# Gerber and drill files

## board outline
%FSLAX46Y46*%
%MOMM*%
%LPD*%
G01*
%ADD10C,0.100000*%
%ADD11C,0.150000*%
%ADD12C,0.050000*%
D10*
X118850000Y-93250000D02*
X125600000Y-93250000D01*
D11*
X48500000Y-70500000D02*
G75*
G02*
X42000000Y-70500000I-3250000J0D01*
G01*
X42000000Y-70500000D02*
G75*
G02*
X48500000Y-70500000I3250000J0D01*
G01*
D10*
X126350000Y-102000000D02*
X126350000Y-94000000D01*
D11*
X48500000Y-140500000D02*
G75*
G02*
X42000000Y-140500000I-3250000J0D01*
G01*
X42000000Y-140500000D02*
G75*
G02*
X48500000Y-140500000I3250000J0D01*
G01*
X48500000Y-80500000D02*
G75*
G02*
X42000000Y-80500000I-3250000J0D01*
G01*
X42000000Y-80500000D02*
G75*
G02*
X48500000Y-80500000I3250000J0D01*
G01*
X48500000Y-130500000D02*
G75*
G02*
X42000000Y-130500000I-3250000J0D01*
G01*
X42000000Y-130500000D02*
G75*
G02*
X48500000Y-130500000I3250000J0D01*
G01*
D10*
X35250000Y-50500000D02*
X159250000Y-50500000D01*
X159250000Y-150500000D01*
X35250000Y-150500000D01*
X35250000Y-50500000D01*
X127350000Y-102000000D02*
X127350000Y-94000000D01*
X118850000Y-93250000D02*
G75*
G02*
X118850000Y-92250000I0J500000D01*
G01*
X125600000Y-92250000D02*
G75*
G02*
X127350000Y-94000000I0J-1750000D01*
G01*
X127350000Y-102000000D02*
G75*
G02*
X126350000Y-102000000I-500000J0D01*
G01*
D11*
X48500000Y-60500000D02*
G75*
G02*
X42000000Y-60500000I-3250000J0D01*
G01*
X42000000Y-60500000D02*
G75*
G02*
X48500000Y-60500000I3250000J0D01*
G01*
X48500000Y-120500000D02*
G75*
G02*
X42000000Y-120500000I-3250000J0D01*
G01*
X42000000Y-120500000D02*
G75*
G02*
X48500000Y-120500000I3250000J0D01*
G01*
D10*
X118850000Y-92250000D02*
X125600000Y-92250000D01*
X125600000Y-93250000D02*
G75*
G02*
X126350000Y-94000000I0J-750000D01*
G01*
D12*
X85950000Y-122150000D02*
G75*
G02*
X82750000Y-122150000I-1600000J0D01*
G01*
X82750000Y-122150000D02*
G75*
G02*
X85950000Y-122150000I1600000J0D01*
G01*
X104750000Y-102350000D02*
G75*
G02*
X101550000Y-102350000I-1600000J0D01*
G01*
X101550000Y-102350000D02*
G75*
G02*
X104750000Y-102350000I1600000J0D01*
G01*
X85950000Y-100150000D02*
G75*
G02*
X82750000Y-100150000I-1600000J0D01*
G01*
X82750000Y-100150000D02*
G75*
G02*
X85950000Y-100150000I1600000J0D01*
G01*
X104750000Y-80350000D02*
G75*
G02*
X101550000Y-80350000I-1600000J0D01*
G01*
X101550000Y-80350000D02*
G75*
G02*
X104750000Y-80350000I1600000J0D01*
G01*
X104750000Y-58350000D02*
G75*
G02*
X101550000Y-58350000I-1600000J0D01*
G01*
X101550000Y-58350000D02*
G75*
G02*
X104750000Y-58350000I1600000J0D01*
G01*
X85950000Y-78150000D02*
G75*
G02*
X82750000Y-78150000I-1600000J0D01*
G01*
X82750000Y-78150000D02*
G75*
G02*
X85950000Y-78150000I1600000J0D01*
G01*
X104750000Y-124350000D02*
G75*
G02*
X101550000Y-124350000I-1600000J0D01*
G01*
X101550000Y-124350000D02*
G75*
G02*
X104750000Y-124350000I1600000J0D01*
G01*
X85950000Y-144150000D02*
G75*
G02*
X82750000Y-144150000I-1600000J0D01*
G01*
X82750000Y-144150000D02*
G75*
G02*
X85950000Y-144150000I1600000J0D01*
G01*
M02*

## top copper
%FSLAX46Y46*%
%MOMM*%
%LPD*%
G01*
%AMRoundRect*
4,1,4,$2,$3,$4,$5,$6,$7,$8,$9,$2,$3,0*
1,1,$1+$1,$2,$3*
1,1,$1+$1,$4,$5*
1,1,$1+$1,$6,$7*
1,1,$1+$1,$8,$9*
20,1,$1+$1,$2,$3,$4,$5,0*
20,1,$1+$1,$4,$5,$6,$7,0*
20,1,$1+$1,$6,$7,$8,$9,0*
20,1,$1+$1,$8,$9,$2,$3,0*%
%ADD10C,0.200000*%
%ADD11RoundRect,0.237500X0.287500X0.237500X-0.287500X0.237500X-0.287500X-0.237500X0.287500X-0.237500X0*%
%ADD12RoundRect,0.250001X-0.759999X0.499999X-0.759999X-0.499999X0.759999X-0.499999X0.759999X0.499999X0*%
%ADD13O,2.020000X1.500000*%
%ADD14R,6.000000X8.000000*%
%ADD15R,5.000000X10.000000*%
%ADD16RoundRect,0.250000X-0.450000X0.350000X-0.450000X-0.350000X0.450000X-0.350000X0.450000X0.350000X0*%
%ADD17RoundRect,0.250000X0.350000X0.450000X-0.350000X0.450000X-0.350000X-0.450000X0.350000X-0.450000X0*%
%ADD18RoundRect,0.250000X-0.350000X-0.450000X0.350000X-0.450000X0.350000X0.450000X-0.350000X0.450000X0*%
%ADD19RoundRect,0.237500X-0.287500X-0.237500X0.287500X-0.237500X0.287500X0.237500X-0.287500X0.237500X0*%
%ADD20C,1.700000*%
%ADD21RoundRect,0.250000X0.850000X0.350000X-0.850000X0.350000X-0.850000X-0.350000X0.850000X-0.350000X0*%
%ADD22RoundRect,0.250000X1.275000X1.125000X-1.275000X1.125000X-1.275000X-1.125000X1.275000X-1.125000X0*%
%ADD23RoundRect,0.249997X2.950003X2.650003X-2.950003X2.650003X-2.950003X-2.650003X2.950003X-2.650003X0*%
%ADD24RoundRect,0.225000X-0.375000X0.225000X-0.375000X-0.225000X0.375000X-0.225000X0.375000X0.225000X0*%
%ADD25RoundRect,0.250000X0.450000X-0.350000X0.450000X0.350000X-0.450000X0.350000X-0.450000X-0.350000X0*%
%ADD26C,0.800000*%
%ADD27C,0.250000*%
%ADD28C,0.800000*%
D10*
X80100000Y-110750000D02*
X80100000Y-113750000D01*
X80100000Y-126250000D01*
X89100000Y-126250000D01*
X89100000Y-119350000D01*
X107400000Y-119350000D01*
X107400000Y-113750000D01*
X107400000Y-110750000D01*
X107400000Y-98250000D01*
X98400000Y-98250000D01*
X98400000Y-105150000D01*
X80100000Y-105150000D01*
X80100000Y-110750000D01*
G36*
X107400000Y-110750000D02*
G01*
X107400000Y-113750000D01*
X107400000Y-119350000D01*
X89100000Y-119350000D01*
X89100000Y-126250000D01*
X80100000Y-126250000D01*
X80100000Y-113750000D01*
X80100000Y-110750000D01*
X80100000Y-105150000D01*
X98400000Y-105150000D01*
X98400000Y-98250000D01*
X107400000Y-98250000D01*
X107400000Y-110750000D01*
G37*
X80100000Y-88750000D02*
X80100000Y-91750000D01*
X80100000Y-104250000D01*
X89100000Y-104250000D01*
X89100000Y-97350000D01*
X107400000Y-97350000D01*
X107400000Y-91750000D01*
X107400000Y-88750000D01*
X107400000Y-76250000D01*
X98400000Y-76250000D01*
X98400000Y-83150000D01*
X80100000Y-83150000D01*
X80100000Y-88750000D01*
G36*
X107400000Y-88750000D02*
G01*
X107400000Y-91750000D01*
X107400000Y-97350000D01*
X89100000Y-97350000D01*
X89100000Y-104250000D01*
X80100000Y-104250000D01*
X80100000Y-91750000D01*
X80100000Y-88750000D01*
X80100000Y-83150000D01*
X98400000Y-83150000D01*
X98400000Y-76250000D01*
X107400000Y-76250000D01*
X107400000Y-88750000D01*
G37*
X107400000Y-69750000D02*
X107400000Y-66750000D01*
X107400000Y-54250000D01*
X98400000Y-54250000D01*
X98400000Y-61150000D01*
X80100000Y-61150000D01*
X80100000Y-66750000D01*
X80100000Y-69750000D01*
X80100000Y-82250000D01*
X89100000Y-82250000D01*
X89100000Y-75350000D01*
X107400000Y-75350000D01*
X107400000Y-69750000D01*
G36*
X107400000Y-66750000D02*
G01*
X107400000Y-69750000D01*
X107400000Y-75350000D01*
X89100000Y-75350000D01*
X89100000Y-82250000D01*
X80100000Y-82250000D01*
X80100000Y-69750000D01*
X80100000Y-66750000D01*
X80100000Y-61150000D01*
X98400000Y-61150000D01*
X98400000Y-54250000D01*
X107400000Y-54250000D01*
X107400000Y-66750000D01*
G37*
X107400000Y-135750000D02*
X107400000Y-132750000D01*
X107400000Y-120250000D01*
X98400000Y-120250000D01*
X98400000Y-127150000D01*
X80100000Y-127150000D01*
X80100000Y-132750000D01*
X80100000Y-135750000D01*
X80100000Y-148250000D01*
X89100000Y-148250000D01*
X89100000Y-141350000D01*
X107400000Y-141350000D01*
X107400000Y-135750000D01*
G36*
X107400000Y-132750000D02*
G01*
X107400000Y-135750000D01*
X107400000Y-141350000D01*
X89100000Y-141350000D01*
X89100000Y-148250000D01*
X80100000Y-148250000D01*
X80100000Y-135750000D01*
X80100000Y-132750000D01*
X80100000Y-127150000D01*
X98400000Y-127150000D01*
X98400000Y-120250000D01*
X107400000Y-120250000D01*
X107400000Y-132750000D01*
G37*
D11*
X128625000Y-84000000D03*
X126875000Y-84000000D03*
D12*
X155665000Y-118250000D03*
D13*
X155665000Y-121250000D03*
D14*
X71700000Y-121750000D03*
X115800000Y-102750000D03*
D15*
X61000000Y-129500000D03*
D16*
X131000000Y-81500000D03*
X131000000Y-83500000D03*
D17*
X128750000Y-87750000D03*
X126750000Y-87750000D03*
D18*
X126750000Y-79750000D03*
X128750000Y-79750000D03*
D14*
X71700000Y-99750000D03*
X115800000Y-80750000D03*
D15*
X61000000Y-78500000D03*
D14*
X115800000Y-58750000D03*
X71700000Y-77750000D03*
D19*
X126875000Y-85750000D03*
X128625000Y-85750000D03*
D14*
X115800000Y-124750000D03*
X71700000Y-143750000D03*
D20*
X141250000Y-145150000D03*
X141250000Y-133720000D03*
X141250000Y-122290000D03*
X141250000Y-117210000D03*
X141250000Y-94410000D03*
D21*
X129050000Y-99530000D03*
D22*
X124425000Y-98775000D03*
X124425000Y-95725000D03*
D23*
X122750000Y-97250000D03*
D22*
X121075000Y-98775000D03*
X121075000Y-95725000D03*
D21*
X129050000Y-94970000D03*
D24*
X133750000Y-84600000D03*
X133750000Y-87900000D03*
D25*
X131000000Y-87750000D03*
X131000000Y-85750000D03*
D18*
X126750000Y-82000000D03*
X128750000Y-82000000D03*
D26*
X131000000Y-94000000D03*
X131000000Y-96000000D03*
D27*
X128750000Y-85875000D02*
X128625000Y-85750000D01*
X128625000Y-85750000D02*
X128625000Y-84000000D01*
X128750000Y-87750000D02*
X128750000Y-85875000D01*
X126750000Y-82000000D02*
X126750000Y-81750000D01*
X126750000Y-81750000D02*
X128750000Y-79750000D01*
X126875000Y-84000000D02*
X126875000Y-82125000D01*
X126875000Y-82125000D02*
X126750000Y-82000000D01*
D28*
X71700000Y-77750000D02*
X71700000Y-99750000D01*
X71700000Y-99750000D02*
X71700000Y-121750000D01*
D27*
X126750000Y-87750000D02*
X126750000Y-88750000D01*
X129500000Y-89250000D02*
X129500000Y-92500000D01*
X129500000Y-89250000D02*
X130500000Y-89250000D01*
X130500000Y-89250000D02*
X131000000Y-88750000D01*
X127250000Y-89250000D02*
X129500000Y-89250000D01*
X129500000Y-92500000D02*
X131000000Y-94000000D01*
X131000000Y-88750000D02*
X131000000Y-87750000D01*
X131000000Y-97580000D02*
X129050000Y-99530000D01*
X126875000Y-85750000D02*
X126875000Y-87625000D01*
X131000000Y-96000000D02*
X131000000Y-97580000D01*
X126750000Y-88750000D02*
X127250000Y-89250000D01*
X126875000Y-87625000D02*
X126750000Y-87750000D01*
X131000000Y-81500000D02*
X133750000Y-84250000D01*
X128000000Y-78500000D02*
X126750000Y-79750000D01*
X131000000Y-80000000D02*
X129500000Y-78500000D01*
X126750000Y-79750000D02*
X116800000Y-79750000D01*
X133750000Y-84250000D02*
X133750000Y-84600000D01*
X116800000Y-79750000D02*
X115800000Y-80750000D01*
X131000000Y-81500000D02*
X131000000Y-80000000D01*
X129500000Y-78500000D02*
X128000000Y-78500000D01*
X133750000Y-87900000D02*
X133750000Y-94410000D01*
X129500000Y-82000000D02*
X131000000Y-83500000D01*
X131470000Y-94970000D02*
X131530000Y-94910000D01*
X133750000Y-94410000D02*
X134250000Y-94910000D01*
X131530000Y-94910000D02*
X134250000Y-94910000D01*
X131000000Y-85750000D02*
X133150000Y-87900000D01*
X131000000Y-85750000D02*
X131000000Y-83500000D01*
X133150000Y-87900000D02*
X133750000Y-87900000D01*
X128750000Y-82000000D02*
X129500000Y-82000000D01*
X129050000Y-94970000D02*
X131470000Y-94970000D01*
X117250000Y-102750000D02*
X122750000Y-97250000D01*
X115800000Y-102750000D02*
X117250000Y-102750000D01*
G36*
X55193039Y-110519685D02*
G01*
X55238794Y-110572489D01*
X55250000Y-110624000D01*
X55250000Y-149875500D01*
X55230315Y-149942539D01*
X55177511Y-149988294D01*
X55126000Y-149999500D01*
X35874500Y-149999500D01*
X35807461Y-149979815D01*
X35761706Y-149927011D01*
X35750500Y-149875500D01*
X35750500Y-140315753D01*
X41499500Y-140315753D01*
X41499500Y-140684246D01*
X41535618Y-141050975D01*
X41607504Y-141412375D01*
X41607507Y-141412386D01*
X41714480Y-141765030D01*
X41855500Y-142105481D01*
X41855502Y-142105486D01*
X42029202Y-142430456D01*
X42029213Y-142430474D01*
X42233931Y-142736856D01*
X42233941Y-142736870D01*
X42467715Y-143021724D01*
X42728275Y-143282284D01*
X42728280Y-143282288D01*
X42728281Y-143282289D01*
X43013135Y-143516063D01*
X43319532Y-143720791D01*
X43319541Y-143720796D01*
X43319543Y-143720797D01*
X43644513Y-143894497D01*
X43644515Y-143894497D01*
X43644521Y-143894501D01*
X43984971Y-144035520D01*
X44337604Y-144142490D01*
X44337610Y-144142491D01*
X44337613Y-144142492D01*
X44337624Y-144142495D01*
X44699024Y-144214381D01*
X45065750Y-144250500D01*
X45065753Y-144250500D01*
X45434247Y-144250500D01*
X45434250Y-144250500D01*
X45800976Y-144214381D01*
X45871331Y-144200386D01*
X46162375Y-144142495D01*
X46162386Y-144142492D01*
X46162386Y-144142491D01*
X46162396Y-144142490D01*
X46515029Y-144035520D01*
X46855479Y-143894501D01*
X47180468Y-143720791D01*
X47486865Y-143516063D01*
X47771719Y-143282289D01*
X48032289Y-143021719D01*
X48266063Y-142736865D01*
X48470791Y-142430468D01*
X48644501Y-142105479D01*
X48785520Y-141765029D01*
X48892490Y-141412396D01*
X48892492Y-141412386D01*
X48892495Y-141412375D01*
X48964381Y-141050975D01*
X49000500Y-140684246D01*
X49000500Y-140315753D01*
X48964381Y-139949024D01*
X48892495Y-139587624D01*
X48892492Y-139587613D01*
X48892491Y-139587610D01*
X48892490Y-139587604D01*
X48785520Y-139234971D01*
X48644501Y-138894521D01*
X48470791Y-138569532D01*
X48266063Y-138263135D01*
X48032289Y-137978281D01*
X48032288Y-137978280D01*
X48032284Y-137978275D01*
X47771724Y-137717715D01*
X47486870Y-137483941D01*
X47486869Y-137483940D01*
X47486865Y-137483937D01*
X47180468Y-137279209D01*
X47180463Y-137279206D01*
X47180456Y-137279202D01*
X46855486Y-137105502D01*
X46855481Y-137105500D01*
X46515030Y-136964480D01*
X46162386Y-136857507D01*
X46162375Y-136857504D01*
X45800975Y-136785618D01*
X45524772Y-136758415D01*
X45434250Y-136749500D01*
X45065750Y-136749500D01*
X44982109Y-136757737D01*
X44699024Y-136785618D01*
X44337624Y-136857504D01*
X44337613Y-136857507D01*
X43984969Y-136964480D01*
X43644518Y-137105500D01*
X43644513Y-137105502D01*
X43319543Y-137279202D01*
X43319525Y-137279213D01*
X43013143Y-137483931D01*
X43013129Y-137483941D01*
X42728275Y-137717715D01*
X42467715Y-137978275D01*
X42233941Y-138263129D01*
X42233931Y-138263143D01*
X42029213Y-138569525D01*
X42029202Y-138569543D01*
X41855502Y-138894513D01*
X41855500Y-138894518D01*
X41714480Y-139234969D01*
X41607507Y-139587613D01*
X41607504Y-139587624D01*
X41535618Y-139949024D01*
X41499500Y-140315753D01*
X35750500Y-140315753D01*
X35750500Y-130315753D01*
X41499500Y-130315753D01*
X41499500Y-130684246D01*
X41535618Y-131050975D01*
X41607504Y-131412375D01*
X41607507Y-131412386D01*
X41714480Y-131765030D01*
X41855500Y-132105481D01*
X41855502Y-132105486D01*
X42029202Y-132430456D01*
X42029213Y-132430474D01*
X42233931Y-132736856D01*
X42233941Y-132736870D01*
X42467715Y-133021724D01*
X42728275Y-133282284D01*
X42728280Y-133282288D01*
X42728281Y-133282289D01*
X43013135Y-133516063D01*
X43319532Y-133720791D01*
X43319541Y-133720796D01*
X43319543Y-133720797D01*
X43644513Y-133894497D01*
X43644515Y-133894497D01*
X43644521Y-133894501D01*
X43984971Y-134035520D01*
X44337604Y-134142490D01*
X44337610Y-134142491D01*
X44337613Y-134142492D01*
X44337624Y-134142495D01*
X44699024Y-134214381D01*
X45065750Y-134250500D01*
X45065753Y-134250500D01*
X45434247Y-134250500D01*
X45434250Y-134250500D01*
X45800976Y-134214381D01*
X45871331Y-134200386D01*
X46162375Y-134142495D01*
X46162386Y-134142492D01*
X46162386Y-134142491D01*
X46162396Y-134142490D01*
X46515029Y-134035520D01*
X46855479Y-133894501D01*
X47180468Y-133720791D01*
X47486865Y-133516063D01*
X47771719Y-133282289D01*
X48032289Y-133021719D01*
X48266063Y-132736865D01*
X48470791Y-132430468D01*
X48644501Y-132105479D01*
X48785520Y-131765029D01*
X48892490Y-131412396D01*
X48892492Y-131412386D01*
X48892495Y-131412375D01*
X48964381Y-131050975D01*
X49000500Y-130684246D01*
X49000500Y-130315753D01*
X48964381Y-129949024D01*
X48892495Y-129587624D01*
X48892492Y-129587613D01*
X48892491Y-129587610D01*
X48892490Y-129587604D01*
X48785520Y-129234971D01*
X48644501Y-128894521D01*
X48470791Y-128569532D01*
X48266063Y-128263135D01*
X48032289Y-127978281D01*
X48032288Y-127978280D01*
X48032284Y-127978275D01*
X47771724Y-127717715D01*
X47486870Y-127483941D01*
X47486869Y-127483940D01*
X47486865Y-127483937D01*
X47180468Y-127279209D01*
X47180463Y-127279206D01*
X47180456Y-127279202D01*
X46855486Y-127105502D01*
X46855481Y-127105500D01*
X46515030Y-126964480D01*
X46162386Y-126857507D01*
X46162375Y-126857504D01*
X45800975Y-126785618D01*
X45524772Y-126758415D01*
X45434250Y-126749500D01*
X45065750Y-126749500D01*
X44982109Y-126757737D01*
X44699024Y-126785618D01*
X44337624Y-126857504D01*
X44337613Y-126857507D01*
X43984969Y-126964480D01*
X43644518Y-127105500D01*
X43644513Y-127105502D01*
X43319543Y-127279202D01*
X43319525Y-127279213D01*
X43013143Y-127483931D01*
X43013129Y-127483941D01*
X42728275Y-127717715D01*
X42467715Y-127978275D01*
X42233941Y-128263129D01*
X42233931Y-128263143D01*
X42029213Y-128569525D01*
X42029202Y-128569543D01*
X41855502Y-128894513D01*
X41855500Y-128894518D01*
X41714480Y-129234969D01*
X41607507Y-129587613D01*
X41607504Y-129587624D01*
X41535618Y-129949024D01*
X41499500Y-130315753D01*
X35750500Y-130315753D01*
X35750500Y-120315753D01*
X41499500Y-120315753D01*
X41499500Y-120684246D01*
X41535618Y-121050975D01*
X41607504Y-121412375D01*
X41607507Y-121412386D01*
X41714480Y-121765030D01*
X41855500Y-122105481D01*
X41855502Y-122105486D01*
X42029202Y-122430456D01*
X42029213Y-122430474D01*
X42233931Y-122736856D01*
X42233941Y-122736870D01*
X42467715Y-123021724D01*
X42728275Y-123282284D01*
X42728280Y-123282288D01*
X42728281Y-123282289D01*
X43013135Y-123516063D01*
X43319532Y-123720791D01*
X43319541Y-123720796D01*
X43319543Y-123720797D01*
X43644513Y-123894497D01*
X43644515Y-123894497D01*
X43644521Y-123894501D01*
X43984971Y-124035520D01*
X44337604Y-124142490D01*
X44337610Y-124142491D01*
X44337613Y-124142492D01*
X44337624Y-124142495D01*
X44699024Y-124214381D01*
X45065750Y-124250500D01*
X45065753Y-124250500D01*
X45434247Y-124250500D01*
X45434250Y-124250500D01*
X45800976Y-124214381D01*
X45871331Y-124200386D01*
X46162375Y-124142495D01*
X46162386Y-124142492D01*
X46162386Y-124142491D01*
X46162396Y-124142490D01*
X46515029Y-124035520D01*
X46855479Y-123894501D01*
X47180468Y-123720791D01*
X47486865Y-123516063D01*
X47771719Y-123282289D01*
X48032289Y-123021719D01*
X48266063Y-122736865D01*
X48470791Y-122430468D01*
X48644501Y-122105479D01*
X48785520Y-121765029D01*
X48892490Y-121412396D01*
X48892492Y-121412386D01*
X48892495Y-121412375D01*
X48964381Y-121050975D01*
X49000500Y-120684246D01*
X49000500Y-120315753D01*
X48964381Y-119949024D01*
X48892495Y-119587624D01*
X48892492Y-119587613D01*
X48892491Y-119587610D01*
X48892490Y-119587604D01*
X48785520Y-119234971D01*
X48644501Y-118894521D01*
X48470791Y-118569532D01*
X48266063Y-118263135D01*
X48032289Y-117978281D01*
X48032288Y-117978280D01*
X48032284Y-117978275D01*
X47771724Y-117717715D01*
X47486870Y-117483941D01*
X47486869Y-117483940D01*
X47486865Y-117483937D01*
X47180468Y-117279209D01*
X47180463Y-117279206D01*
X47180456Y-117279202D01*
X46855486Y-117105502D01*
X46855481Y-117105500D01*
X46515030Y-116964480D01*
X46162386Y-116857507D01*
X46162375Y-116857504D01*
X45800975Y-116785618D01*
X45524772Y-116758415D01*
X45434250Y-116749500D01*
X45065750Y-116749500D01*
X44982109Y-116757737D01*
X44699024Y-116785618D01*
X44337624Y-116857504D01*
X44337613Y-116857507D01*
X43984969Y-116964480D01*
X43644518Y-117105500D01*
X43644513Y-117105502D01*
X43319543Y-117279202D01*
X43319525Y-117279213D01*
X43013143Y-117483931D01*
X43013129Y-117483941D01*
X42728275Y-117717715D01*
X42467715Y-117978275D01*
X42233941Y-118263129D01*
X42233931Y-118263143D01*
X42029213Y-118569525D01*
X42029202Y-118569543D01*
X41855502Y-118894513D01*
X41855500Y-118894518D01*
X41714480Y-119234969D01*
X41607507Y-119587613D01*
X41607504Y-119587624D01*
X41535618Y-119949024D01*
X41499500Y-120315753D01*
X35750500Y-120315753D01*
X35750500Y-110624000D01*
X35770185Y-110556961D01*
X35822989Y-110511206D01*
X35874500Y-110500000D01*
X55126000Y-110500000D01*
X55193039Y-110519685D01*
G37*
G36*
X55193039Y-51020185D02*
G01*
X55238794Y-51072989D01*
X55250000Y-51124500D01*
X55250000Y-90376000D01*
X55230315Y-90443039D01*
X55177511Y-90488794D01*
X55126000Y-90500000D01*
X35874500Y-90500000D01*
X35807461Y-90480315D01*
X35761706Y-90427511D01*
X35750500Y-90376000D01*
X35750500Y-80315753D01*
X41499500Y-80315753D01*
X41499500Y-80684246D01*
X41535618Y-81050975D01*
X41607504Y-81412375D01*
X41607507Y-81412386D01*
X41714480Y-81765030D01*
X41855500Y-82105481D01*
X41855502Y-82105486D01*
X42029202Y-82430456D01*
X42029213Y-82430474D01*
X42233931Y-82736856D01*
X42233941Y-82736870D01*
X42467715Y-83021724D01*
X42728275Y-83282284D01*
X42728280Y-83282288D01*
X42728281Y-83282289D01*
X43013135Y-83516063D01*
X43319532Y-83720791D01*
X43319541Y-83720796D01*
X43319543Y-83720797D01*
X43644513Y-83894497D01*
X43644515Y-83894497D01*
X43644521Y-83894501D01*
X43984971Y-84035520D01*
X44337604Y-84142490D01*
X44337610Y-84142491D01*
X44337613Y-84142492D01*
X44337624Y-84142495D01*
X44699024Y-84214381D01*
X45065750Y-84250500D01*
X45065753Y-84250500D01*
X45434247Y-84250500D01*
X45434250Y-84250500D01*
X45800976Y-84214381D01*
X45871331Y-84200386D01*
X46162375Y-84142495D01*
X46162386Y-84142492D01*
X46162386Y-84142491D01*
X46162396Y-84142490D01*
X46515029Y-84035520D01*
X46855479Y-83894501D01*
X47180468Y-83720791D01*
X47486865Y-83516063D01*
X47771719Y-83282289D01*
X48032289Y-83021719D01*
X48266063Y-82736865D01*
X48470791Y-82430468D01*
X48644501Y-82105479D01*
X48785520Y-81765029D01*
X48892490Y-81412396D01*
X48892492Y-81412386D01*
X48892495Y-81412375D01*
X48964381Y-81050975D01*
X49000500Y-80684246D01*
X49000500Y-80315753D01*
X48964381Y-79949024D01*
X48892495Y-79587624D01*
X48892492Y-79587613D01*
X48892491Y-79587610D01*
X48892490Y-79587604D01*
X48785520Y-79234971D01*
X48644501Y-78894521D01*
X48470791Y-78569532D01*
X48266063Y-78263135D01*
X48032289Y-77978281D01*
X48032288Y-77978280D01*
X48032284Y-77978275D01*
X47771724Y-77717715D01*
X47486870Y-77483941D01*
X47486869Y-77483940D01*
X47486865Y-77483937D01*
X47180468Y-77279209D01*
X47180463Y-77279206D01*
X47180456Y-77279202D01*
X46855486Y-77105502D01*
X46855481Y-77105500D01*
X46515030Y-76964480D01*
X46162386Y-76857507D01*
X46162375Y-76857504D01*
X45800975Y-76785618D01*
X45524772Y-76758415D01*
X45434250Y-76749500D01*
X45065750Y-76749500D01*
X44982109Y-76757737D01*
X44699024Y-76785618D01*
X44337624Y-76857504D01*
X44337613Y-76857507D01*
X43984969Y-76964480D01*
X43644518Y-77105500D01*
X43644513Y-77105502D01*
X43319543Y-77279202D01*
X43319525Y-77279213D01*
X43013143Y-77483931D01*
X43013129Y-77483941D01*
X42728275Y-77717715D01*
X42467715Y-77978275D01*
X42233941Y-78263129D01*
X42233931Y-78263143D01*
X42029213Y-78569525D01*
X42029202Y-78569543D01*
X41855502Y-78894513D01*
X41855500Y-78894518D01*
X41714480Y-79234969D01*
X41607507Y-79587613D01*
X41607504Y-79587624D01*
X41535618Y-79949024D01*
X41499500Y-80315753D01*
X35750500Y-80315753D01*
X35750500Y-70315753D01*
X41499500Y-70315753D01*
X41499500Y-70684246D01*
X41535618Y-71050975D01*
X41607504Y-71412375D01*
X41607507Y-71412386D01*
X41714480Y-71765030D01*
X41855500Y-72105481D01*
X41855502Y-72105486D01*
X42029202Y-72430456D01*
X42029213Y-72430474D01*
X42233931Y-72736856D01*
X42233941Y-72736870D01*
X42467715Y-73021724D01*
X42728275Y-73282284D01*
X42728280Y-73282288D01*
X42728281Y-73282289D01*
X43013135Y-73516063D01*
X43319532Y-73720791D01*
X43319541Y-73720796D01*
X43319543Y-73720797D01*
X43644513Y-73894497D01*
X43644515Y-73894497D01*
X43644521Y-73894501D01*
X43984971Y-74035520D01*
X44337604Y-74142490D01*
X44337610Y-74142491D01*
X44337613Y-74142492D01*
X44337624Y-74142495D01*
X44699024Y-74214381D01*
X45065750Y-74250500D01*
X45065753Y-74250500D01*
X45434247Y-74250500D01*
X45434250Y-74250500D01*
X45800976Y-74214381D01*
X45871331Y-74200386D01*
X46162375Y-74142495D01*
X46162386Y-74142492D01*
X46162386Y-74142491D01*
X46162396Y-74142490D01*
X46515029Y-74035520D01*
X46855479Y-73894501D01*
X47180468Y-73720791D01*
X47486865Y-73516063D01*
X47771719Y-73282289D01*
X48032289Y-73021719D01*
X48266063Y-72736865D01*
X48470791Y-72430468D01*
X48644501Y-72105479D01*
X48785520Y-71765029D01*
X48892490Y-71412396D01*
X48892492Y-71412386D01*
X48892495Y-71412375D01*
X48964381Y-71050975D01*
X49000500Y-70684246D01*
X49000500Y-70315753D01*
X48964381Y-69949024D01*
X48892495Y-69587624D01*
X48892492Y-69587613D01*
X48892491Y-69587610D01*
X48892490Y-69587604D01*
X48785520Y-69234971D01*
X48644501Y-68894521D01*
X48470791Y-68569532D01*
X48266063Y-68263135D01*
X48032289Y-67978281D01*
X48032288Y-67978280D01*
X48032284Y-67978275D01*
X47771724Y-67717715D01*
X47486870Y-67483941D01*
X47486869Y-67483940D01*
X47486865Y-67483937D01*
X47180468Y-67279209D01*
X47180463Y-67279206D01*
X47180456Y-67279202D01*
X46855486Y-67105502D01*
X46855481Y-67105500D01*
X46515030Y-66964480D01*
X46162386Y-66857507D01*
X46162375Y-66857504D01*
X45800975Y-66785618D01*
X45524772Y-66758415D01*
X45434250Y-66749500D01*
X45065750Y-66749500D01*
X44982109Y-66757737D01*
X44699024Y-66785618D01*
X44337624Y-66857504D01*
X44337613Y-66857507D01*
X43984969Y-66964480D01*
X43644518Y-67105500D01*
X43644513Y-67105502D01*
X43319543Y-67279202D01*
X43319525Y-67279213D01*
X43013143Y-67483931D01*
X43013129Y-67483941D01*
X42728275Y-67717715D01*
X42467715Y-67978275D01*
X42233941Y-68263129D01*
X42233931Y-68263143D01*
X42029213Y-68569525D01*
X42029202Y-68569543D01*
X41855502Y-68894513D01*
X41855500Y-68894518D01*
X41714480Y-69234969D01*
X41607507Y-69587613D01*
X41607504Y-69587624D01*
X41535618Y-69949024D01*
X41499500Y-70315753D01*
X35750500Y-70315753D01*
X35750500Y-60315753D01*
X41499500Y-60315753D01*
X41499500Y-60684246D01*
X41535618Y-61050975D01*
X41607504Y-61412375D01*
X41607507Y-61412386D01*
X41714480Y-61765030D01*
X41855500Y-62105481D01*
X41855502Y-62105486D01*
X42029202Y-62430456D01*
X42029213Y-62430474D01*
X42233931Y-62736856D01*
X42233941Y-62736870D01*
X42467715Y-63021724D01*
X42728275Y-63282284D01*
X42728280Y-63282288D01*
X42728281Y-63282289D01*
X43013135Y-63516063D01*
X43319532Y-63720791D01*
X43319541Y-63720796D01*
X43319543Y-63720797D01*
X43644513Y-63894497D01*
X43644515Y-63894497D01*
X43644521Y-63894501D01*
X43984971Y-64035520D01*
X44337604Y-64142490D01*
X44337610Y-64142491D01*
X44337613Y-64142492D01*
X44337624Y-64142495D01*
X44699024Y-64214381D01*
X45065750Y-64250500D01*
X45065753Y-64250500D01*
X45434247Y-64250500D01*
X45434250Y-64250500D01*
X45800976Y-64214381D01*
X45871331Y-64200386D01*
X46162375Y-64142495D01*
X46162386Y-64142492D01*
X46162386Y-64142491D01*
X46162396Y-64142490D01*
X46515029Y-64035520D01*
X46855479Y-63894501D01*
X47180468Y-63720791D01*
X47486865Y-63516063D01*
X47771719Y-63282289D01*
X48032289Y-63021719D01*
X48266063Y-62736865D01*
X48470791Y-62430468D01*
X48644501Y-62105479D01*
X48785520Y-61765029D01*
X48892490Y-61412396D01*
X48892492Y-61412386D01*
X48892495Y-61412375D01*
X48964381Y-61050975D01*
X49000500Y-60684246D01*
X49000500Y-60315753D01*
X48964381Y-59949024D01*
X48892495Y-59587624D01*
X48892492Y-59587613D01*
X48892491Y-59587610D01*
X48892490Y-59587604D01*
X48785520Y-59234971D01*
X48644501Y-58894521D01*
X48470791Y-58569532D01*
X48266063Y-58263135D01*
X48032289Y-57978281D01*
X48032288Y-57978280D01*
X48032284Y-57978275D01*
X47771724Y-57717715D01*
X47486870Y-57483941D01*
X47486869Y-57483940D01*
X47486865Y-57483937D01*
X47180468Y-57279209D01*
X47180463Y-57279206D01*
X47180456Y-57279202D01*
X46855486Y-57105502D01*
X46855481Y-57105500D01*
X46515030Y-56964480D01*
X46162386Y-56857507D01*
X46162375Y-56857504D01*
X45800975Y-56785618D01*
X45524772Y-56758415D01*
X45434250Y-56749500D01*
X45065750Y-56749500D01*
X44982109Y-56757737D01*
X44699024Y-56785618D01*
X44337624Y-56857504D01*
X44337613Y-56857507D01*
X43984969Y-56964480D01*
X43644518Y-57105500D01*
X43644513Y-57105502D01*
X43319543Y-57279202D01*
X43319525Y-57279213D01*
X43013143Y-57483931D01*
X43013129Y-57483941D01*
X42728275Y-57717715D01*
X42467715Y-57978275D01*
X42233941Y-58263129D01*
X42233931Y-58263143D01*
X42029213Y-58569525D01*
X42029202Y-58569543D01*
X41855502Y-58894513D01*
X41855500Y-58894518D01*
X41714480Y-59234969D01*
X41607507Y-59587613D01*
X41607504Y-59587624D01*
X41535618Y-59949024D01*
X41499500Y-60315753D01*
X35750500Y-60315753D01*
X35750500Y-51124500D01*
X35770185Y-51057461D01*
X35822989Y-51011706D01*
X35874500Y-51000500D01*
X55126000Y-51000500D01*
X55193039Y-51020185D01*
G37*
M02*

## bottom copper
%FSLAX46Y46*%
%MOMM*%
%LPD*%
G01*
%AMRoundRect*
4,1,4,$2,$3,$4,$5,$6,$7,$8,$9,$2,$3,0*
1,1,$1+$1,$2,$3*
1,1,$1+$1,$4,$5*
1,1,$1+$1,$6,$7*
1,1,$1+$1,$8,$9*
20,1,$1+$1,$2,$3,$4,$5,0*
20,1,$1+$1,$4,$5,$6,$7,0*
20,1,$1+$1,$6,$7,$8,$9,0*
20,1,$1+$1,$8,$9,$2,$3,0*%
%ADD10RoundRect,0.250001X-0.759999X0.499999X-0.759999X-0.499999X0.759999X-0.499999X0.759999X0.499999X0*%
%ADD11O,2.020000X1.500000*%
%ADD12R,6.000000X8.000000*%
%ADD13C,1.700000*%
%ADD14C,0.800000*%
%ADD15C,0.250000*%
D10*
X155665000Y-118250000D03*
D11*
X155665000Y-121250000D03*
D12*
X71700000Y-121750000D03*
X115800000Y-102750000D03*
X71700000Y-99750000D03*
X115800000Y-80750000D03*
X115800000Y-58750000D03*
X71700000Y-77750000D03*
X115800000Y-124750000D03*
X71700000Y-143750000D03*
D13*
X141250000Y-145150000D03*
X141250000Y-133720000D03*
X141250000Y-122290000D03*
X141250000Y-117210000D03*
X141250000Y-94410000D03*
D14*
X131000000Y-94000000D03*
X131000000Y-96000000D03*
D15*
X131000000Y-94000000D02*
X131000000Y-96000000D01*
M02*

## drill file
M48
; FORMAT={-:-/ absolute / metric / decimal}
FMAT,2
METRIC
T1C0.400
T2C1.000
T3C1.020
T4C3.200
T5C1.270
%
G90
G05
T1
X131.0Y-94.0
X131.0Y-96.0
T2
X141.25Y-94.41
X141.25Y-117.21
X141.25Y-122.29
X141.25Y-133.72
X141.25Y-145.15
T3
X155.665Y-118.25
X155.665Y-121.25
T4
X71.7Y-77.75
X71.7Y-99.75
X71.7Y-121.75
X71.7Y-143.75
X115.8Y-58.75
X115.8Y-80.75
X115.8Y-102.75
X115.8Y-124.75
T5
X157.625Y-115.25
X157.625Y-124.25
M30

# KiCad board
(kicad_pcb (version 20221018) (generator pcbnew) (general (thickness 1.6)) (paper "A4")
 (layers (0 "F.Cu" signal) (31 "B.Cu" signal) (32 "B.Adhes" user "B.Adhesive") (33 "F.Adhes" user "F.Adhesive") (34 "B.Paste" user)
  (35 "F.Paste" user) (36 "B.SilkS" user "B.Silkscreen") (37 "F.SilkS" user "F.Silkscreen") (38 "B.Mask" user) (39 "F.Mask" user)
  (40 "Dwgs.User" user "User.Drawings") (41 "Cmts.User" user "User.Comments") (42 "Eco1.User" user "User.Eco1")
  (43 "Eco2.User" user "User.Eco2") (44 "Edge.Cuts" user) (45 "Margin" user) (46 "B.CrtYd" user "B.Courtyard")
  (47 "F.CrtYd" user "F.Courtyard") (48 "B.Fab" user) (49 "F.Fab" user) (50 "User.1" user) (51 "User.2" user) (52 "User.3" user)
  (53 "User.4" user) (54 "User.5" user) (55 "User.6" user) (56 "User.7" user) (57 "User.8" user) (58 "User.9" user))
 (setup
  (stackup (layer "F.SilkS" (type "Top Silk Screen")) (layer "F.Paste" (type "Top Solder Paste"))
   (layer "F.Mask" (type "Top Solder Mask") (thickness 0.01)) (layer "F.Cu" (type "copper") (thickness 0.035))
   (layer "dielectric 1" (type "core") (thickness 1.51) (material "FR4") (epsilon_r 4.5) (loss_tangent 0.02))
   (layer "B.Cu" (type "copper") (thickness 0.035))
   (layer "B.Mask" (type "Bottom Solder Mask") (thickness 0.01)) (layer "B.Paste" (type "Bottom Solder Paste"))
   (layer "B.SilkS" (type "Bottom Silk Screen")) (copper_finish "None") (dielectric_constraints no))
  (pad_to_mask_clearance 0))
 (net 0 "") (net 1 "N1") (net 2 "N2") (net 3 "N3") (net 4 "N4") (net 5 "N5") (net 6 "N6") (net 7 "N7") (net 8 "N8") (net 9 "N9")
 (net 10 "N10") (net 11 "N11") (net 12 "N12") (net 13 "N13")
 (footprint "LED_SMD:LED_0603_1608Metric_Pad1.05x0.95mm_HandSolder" (layer "F.Cu") (at 127.75 84 180)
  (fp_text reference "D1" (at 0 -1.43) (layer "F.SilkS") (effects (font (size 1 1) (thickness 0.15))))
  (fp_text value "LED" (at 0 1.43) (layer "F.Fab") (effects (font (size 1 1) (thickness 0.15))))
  (pad "1" smd roundrect (at -0.875 0 180) (size 1.05 0.95) (layers "F.Cu" "F.Paste" "F.Mask") (roundrect_rratio 0.25) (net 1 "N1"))
  (pad "2" smd roundrect (at 0.875 0 180) (size 1.05 0.95) (layers "F.Cu" "F.Paste" "F.Mask") (roundrect_rratio 0.25) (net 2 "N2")))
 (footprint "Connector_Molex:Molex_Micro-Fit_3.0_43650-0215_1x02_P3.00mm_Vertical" (layer "F.Cu") (at 155.665 118.25 -90)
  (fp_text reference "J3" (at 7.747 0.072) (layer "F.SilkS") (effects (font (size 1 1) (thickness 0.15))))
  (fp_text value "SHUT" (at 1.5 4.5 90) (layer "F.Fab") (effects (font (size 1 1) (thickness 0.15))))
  (pad "" np_thru_hole circle (at -3 -1.96 270) (size 1.27 1.27) (drill 1.27) (layers "*.Cu" "*.Mask"))
  (pad "" np_thru_hole circle (at 6 -1.96 270) (size 1.27 1.27) (drill 1.27) (layers "*.Cu" "*.Mask"))
  (pad "1" thru_hole roundrect (at 0 0 270) (size 1.5 2.02) (drill 1.02) (layers "*.Cu" "*.Mask") (roundrect_rratio 0.166667) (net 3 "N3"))
  (pad "2" thru_hole oval (at 3 0 270) (size 1.5 2.02) (drill 1.02) (layers "*.Cu" "*.Mask") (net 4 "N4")))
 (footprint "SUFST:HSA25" (layer "F.Cu") (at 93.75 112.25)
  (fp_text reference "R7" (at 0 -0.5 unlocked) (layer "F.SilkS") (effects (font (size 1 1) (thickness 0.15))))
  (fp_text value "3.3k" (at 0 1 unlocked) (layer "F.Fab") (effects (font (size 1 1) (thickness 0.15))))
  (fp_poly
   (pts (xy -13.65 -1.5) (xy -13.65 1.5) (xy -13.65 14) (xy -4.65 14) (xy -4.65 7.1) (xy 13.65 7.1) (xy 13.65 1.5) (xy 13.65 -1.5)
    (xy 13.65 -14) (xy 4.65 -14) (xy 4.65 -7.1) (xy -13.65 -7.1) (xy -13.65 -1.5))
   (stroke (width 0.2) (type solid)) (fill solid) (layer "F.Cu"))
  (fp_circle (center -9.4 9.9) (end -7.8 9.9) (stroke (width 0.05) (type default)) (fill none) (layer "Edge.Cuts"))
  (fp_circle (center 9.4 -9.9) (end 11 -9.9) (stroke (width 0.05) (type default)) (fill none) (layer "Edge.Cuts"))
  (pad "1" thru_hole rect (at -22.05 9.5 90) (size 8 6) (drill 3.2) (layers "*.Cu" "*.Mask") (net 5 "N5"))
  (pad "2" thru_hole rect (at 22.05 -9.5 90) (size 8 6) (drill 3.2) (layers "*.Cu" "*.Mask") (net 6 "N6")))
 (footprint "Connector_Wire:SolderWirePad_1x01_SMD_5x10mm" (layer "F.Cu") (at 61 129.5)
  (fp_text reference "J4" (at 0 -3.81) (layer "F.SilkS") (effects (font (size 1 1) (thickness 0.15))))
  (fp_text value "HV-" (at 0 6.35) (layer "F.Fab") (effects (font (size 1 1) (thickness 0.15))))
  (pad "1" smd rect (at 0 0) (size 5 10) (layers "F.Cu" "F.Paste" "F.Mask") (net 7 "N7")))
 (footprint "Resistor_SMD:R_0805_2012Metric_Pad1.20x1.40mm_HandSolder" (layer "F.Cu") (at 131 82.5 -90)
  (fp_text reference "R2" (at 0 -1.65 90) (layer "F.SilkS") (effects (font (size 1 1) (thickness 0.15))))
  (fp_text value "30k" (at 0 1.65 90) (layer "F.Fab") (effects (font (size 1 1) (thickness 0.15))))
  (pad "1" smd roundrect (at -1 0 270) (size 1.2 1.4) (layers "F.Cu" "F.Paste" "F.Mask") (roundrect_rratio 0.208333) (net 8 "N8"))
  (pad "2" smd roundrect (at 1 0 270) (size 1.2 1.4) (layers "F.Cu" "F.Paste" "F.Mask") (roundrect_rratio 0.208333) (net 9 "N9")))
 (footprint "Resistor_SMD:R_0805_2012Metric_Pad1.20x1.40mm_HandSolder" (layer "F.Cu") (at 127.75 87.75 180)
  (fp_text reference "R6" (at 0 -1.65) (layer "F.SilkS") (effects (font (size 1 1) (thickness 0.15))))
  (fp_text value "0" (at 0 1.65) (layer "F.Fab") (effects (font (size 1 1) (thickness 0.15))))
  (pad "1" smd roundrect (at -1 0 180) (size 1.2 1.4) (layers "F.Cu" "F.Paste" "F.Mask") (roundrect_rratio 0.208333) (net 1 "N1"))
  (pad "2" smd roundrect (at 1 0 180) (size 1.2 1.4) (layers "F.Cu" "F.Paste" "F.Mask") (roundrect_rratio 0.208333) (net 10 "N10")))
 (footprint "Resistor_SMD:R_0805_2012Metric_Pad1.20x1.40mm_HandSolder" (layer "F.Cu") (at 127.75 79.75)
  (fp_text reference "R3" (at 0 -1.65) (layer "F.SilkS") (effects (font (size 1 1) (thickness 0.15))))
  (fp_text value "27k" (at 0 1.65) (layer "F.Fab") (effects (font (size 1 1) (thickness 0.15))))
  (pad "1" smd roundrect (at -1 0) (size 1.2 1.4) (layers "F.Cu" "F.Paste" "F.Mask") (roundrect_rratio 0.208333) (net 8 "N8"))
  (pad "2" smd roundrect (at 1 0) (size 1.2 1.4) (layers "F.Cu" "F.Paste" "F.Mask") (roundrect_rratio 0.208333) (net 2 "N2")))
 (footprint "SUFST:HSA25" (layer "F.Cu") (at 93.75 90.25)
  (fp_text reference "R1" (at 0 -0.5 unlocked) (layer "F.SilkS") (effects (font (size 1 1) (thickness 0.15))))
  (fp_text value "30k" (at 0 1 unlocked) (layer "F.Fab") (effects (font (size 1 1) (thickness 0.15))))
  (fp_poly
   (pts (xy -13.65 -1.5) (xy -13.65 1.5) (xy -13.65 14) (xy -4.65 14) (xy -4.65 7.1) (xy 13.65 7.1) (xy 13.65 1.5) (xy 13.65 -1.5)
    (xy 13.65 -14) (xy 4.65 -14) (xy 4.65 -7.1) (xy -13.65 -7.1) (xy -13.65 -1.5))
   (stroke (width 0.2) (type solid)) (fill solid) (layer "F.Cu"))
  (fp_circle (center -9.4 9.9) (end -7.8 9.9) (stroke (width 0.05) (type default)) (fill none) (layer "Edge.Cuts"))
  (fp_circle (center 9.4 -9.9) (end 11 -9.9) (stroke (width 0.05) (type default)) (fill none) (layer "Edge.Cuts"))
  (pad "1" thru_hole rect (at -22.05 9.5 90) (size 8 6) (drill 3.2) (layers "*.Cu" "*.Mask") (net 5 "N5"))
  (pad "2" thru_hole rect (at 22.05 -9.5 90) (size 8 6) (drill 3.2) (layers "*.Cu" "*.Mask") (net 8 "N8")))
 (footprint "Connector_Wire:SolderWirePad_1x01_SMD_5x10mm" (layer "F.Cu") (at 61 78.5 180)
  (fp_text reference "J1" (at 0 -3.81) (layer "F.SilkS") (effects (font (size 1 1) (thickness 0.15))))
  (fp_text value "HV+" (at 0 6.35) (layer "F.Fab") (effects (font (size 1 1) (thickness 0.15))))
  (pad "1" smd rect (at 0 0 180) (size 5 10) (layers "F.Cu" "F.Paste" "F.Mask") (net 5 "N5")))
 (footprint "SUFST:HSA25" (layer "F.Cu") (at 93.75 68.25 180)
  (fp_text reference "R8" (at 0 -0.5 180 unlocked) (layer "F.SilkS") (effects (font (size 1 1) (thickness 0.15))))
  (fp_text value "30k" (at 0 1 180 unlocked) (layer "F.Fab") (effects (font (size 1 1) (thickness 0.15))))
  (fp_poly
   (pts (xy -13.65 -1.5) (xy -13.65 1.5) (xy -13.65 14) (xy -4.65 14) (xy -4.65 7.1) (xy 13.65 7.1) (xy 13.65 1.5) (xy 13.65 -1.5)
    (xy 13.65 -14) (xy 4.65 -14) (xy 4.65 -7.1) (xy -13.65 -7.1) (xy -13.65 -1.5))
   (stroke (width 0.2) (type solid)) (fill solid) (layer "F.Cu"))
  (fp_circle (center -9.4 9.9) (end -7.8 9.9) (stroke (width 0.05) (type default)) (fill none) (layer "Edge.Cuts"))
  (fp_circle (center 9.4 -9.9) (end 11 -9.9) (stroke (width 0.05) (type default)) (fill none) (layer "Edge.Cuts"))
  (pad "1" thru_hole rect (at -22.05 9.5 270) (size 8 6) (drill 3.2) (layers "*.Cu" "*.Mask") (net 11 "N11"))
  (pad "2" thru_hole rect (at 22.05 -9.5 270) (size 8 6) (drill 3.2) (layers "*.Cu" "*.Mask") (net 5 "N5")))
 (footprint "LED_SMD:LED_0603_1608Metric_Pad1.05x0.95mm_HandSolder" (layer "F.Cu") (at 127.75 85.75)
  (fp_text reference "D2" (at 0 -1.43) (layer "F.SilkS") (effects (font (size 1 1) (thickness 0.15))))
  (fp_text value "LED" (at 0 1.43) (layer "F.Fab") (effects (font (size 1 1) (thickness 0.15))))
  (pad "1" smd roundrect (at -0.875 0) (size 1.05 0.95) (layers "F.Cu" "F.Paste" "F.Mask") (roundrect_rratio 0.25) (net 10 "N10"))
  (pad "2" smd roundrect (at 0.875 0) (size 1.05 0.95) (layers "F.Cu" "F.Paste" "F.Mask") (roundrect_rratio 0.25) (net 1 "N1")))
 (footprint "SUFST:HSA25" (layer "F.Cu") (at 93.75 134.25 180)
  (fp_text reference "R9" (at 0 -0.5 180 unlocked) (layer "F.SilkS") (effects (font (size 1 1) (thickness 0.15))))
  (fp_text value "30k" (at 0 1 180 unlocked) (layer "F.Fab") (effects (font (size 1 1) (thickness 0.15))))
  (fp_poly
   (pts (xy -13.65 -1.5) (xy -13.65 1.5) (xy -13.65 14) (xy -4.65 14) (xy -4.65 7.1) (xy 13.65 7.1) (xy 13.65 1.5) (xy 13.65 -1.5)
    (xy 13.65 -14) (xy 4.65 -14) (xy 4.65 -7.1) (xy -13.65 -7.1) (xy -13.65 -1.5))
   (stroke (width 0.2) (type solid)) (fill solid) (layer "F.Cu"))
  (fp_circle (center -9.4 9.9) (end -7.8 9.9) (stroke (width 0.05) (type default)) (fill none) (layer "Edge.Cuts"))
  (fp_circle (center 9.4 -9.9) (end 11 -9.9) (stroke (width 0.05) (type default)) (fill none) (layer "Edge.Cuts"))
  (pad "1" thru_hole rect (at -22.05 9.5 270) (size 8 6) (drill 3.2) (layers "*.Cu" "*.Mask") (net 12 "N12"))
  (pad "2" thru_hole rect (at 22.05 -9.5 270) (size 8 6) (drill 3.2) (layers "*.Cu" "*.Mask") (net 7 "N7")))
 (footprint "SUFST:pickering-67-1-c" (layer "F.Cu") (at 141.25 119.75 90)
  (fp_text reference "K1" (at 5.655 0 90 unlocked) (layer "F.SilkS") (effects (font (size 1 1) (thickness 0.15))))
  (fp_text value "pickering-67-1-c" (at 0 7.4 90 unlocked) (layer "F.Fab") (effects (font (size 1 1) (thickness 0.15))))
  (pad "1" thru_hole circle (at -25.4 0 90) (size 1.7 1.7) (drill 1) (layers "*.Cu" "*.Mask") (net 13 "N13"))
  (pad "2" thru_hole circle (at -13.97 0 90) (size 1.7 1.7) (drill 1) (layers "*.Cu" "*.Mask") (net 7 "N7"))
  (pad "3" thru_hole circle (at -2.54 0 90) (size 1.7 1.7) (drill 1) (layers "*.Cu" "*.Mask") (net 4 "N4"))
  (pad "5" thru_hole circle (at 2.54 0 90) (size 1.7 1.7) (drill 1) (layers "*.Cu" "*.Mask") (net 3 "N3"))
  (pad "7" thru_hole circle (at 25.34 0 90) (size 1.7 1.7) (drill 1) (layers "*.Cu" "*.Mask") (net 9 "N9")))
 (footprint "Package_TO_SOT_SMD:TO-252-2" (layer "F.Cu") (at 124.01 97.25 180)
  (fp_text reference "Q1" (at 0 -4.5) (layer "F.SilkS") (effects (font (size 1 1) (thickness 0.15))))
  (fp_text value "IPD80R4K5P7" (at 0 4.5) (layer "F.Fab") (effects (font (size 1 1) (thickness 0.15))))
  (pad "1" smd roundrect (at -5.04 -2.28 180) (size 2.2 1.2) (layers "F.Cu" "F.Paste" "F.Mask") (roundrect_rratio 0.208333) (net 10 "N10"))
  (pad "2" smd roundrect (at -0.415 -1.525 180) (size 3.05 2.75) (layers "F.Cu" "F.Paste") (roundrect_rratio 0.090909) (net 6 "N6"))
  (pad "2" smd roundrect (at -0.415 1.525 180) (size 3.05 2.75) (layers "F.Cu" "F.Paste") (roundrect_rratio 0.090909) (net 6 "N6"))
  (pad "2" smd roundrect (at 1.26 0 180) (size 6.4 5.8) (layers "F.Cu" "F.Mask") (roundrect_rratio 0.043103) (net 6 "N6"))
  (pad "2" smd roundrect (at 2.935 -1.525 180) (size 3.05 2.75) (layers "F.Cu" "F.Paste") (roundrect_rratio 0.090909) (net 6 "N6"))
  (pad "2" smd roundrect (at 2.935 1.525 180) (size 3.05 2.75) (layers "F.Cu" "F.Paste") (roundrect_rratio 0.090909) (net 6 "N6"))
  (pad "3" smd roundrect (at -5.04 2.28 180) (size 2.2 1.2) (layers "F.Cu" "F.Paste" "F.Mask") (roundrect_rratio 0.208333) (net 9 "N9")))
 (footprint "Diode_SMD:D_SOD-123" (layer "F.Cu") (at 133.75 86.25 -90)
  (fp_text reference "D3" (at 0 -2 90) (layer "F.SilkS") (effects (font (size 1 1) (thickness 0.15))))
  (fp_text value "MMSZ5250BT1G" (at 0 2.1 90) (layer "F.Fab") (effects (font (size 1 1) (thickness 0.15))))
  (pad "1" smd roundrect (at -1.65 0 270) (size 0.9 1.2) (layers "F.Cu" "F.Paste" "F.Mask") (roundrect_rratio 0.25) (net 8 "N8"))
  (pad "2" smd roundrect (at 1.65 0 270) (size 0.9 1.2) (layers "F.Cu" "F.Paste" "F.Mask") (roundrect_rratio 0.25) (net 9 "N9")))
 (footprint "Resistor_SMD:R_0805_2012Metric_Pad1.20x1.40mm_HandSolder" (layer "F.Cu") (at 131 86.75 90)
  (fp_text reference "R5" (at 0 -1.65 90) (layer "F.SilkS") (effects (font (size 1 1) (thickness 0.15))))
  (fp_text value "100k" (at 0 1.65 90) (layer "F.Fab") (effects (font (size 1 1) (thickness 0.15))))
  (pad "1" smd roundrect (at -1 0 90) (size 1.2 1.4) (layers "F.Cu" "F.Paste" "F.Mask") (roundrect_rratio 0.208333) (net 10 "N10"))
  (pad "2" smd roundrect (at 1 0 90) (size 1.2 1.4) (layers "F.Cu" "F.Paste" "F.Mask") (roundrect_rratio 0.208333) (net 9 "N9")))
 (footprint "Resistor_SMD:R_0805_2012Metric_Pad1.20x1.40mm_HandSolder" (layer "F.Cu") (at 127.75 82)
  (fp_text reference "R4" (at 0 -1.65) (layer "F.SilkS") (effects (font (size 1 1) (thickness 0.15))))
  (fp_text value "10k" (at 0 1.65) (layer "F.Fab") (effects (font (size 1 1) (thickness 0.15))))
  (pad "1" smd roundrect (at -1 0) (size 1.2 1.4) (layers "F.Cu" "F.Paste" "F.Mask") (roundrect_rratio 0.208333) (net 2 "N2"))
  (pad "2" smd roundrect (at 1 0) (size 1.2 1.4) (layers "F.Cu" "F.Paste" "F.Mask") (roundrect_rratio 0.208333) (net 9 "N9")))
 (gr_line (start 118.85 93.25) (end 125.6 93.25) (stroke (width 0.1) (type default)) (layer "Edge.Cuts"))
 (gr_circle (center 45.25 70.5) (end 48.5 70.5) (stroke (width 0.15) (type default)) (fill none) (layer "Edge.Cuts"))
 (gr_line (start 126.35 102) (end 126.35 94) (stroke (width 0.1) (type default)) (layer "Edge.Cuts"))
 (gr_circle (center 45.25 140.5) (end 48.5 140.5) (stroke (width 0.15) (type default)) (fill none) (layer "Edge.Cuts"))
 (gr_circle (center 45.25 80.5) (end 48.5 80.5) (stroke (width 0.15) (type default)) (fill none) (layer "Edge.Cuts"))
 (gr_circle (center 45.25 130.5) (end 48.5 130.5) (stroke (width 0.15) (type default)) (fill none) (layer "Edge.Cuts"))
 (gr_rect (start 35.25 50.5) (end 159.25 150.5) (stroke (width 0.1) (type default)) (fill none) (layer "Edge.Cuts"))
 (gr_line (start 127.35 102) (end 127.35 94) (stroke (width 0.1) (type default)) (layer "Edge.Cuts"))
 (gr_arc (start 118.85 93.25) (mid 118.35 92.75) (end 118.85 92.25) (stroke (width 0.1) (type default)) (layer "Edge.Cuts"))
 (gr_arc (start 125.6 92.25) (mid 126.837437 92.762563) (end 127.35 94) (stroke (width 0.1) (type default)) (layer "Edge.Cuts"))
 (gr_arc (start 127.35 102) (mid 126.85 102.5) (end 126.35 102) (stroke (width 0.1) (type default)) (layer "Edge.Cuts"))
 (gr_circle (center 45.25 60.5) (end 48.5 60.5) (stroke (width 0.15) (type default)) (fill none) (layer "Edge.Cuts"))
 (gr_circle (center 45.25 120.5) (end 48.5 120.5) (stroke (width 0.15) (type default)) (fill none) (layer "Edge.Cuts"))
 (gr_line (start 118.85 92.25) (end 125.6 92.25) (stroke (width 0.1) (type default)) (layer "Edge.Cuts"))
 (gr_arc (start 125.6 93.25) (mid 126.13033 93.46967) (end 126.35 94) (stroke (width 0.1) (type default)) (layer "Edge.Cuts"))
 (segment (start 128.75 85.875) (end 128.625 85.75) (width 0.25) (layer "F.Cu") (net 1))
 (segment (start 128.625 85.75) (end 128.625 84) (width 0.25) (layer "F.Cu") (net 1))
 (segment (start 128.75 87.75) (end 128.75 85.875) (width 0.25) (layer "F.Cu") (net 1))
 (segment (start 126.75 82) (end 126.75 81.75) (width 0.25) (layer "F.Cu") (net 2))
 (segment (start 126.75 81.75) (end 128.75 79.75) (width 0.25) (layer "F.Cu") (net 2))
 (segment (start 126.875 84) (end 126.875 82.125) (width 0.25) (layer "F.Cu") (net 2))
 (segment (start 126.875 82.125) (end 126.75 82) (width 0.25) (layer "F.Cu") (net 2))
 (segment (start 71.7 77.75) (end 71.7 99.75) (width 0.8) (layer "F.Cu") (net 5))
 (segment (start 71.7 99.75) (end 71.7 121.75) (width 0.8) (layer "F.Cu") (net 5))
 (segment (start 126.75 87.75) (end 126.75 88.75) (width 0.25) (layer "F.Cu") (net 10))
 (segment (start 129.5 89.25) (end 129.5 92.5) (width 0.25) (layer "F.Cu") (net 10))
 (segment (start 129.5 89.25) (end 130.5 89.25) (width 0.25) (layer "F.Cu") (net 10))
 (segment (start 130.5 89.25) (end 131 88.75) (width 0.25) (layer "F.Cu") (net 10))
 (segment (start 127.25 89.25) (end 129.5 89.25) (width 0.25) (layer "F.Cu") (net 10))
 (segment (start 129.5 92.5) (end 131 94) (width 0.25) (layer "F.Cu") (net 10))
 (segment (start 131 88.75) (end 131 87.75) (width 0.25) (layer "F.Cu") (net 10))
 (segment (start 131 97.58) (end 129.05 99.53) (width 0.25) (layer "F.Cu") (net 10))
 (segment (start 126.875 85.75) (end 126.875 87.625) (width 0.25) (layer "F.Cu") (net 10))
 (segment (start 131 96) (end 131 97.58) (width 0.25) (layer "F.Cu") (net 10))
 (segment (start 126.75 88.75) (end 127.25 89.25) (width 0.25) (layer "F.Cu") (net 10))
 (segment (start 126.875 87.625) (end 126.75 87.75) (width 0.25) (layer "F.Cu") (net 10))
 (via (at 131 94) (size 0.8) (drill 0.4) (layers "F.Cu" "B.Cu") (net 10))
 (via (at 131 96) (size 0.8) (drill 0.4) (layers "F.Cu" "B.Cu") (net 10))
 (segment (start 131 94) (end 131 96) (width 0.25) (layer "B.Cu") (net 10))
 (segment (start 131 81.5) (end 133.75 84.25) (width 0.25) (layer "F.Cu") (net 8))
 (segment (start 128 78.5) (end 126.75 79.75) (width 0.25) (layer "F.Cu") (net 8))
 (segment (start 131 80) (end 129.5 78.5) (width 0.25) (layer "F.Cu") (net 8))
 (segment (start 126.75 79.75) (end 116.8 79.75) (width 0.25) (layer "F.Cu") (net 8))
 (segment (start 133.75 84.25) (end 133.75 84.6) (width 0.25) (layer "F.Cu") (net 8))
 (segment (start 116.8 79.75) (end 115.8 80.75) (width 0.25) (layer "F.Cu") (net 8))
 (segment (start 131 81.5) (end 131 80) (width 0.25) (layer "F.Cu") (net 8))
 (segment (start 129.5 78.5) (end 128 78.5) (width 0.25) (layer "F.Cu") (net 8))
 (segment (start 133.75 87.9) (end 133.75 94.41) (width 0.25) (layer "F.Cu") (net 9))
 (segment (start 129.5 82) (end 131 83.5) (width 0.25) (layer "F.Cu") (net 9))
 (segment (start 131.47 94.97) (end 131.53 94.91) (width 0.25) (layer "F.Cu") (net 9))
 (segment (start 133.75 94.41) (end 134.25 94.91) (width 0.25) (layer "F.Cu") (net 9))
 (segment (start 131.53 94.91) (end 134.25 94.91) (width 0.25) (layer "F.Cu") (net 9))
 (segment (start 131 85.75) (end 133.15 87.9) (width 0.25) (layer "F.Cu") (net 9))
 (segment (start 131 85.75) (end 131 83.5) (width 0.25) (layer "F.Cu") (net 9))
 (segment (start 133.15 87.9) (end 133.75 87.9) (width 0.25) (layer "F.Cu") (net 9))
 (segment (start 128.75 82) (end 129.5 82) (width 0.25) (layer "F.Cu") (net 9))
 (segment (start 129.05 94.97) (end 131.47 94.97) (width 0.25) (layer "F.Cu") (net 9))
 (segment (start 117.25 102.75) (end 122.75 97.25) (width 0.25) (layer "F.Cu") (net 6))
 (segment (start 115.8 102.75) (end 117.25 102.75) (width 0.25) (layer "F.Cu") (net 6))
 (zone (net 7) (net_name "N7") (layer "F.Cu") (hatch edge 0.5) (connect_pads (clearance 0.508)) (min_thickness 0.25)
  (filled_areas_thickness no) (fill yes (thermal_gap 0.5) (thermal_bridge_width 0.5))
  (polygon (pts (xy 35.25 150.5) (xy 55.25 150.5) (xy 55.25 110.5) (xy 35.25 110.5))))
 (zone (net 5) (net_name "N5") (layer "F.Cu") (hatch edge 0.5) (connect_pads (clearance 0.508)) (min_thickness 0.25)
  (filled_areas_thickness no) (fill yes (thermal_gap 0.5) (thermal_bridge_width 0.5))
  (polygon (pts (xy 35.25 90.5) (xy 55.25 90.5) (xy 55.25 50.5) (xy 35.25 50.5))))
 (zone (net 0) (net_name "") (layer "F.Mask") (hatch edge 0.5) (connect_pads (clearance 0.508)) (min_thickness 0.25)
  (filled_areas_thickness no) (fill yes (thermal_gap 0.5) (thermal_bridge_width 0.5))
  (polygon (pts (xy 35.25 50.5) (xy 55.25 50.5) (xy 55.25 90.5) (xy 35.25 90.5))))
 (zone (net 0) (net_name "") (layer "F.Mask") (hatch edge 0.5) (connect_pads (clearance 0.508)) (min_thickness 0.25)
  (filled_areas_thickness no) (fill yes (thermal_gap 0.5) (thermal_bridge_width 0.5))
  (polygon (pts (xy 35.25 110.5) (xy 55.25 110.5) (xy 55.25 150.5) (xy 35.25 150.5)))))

